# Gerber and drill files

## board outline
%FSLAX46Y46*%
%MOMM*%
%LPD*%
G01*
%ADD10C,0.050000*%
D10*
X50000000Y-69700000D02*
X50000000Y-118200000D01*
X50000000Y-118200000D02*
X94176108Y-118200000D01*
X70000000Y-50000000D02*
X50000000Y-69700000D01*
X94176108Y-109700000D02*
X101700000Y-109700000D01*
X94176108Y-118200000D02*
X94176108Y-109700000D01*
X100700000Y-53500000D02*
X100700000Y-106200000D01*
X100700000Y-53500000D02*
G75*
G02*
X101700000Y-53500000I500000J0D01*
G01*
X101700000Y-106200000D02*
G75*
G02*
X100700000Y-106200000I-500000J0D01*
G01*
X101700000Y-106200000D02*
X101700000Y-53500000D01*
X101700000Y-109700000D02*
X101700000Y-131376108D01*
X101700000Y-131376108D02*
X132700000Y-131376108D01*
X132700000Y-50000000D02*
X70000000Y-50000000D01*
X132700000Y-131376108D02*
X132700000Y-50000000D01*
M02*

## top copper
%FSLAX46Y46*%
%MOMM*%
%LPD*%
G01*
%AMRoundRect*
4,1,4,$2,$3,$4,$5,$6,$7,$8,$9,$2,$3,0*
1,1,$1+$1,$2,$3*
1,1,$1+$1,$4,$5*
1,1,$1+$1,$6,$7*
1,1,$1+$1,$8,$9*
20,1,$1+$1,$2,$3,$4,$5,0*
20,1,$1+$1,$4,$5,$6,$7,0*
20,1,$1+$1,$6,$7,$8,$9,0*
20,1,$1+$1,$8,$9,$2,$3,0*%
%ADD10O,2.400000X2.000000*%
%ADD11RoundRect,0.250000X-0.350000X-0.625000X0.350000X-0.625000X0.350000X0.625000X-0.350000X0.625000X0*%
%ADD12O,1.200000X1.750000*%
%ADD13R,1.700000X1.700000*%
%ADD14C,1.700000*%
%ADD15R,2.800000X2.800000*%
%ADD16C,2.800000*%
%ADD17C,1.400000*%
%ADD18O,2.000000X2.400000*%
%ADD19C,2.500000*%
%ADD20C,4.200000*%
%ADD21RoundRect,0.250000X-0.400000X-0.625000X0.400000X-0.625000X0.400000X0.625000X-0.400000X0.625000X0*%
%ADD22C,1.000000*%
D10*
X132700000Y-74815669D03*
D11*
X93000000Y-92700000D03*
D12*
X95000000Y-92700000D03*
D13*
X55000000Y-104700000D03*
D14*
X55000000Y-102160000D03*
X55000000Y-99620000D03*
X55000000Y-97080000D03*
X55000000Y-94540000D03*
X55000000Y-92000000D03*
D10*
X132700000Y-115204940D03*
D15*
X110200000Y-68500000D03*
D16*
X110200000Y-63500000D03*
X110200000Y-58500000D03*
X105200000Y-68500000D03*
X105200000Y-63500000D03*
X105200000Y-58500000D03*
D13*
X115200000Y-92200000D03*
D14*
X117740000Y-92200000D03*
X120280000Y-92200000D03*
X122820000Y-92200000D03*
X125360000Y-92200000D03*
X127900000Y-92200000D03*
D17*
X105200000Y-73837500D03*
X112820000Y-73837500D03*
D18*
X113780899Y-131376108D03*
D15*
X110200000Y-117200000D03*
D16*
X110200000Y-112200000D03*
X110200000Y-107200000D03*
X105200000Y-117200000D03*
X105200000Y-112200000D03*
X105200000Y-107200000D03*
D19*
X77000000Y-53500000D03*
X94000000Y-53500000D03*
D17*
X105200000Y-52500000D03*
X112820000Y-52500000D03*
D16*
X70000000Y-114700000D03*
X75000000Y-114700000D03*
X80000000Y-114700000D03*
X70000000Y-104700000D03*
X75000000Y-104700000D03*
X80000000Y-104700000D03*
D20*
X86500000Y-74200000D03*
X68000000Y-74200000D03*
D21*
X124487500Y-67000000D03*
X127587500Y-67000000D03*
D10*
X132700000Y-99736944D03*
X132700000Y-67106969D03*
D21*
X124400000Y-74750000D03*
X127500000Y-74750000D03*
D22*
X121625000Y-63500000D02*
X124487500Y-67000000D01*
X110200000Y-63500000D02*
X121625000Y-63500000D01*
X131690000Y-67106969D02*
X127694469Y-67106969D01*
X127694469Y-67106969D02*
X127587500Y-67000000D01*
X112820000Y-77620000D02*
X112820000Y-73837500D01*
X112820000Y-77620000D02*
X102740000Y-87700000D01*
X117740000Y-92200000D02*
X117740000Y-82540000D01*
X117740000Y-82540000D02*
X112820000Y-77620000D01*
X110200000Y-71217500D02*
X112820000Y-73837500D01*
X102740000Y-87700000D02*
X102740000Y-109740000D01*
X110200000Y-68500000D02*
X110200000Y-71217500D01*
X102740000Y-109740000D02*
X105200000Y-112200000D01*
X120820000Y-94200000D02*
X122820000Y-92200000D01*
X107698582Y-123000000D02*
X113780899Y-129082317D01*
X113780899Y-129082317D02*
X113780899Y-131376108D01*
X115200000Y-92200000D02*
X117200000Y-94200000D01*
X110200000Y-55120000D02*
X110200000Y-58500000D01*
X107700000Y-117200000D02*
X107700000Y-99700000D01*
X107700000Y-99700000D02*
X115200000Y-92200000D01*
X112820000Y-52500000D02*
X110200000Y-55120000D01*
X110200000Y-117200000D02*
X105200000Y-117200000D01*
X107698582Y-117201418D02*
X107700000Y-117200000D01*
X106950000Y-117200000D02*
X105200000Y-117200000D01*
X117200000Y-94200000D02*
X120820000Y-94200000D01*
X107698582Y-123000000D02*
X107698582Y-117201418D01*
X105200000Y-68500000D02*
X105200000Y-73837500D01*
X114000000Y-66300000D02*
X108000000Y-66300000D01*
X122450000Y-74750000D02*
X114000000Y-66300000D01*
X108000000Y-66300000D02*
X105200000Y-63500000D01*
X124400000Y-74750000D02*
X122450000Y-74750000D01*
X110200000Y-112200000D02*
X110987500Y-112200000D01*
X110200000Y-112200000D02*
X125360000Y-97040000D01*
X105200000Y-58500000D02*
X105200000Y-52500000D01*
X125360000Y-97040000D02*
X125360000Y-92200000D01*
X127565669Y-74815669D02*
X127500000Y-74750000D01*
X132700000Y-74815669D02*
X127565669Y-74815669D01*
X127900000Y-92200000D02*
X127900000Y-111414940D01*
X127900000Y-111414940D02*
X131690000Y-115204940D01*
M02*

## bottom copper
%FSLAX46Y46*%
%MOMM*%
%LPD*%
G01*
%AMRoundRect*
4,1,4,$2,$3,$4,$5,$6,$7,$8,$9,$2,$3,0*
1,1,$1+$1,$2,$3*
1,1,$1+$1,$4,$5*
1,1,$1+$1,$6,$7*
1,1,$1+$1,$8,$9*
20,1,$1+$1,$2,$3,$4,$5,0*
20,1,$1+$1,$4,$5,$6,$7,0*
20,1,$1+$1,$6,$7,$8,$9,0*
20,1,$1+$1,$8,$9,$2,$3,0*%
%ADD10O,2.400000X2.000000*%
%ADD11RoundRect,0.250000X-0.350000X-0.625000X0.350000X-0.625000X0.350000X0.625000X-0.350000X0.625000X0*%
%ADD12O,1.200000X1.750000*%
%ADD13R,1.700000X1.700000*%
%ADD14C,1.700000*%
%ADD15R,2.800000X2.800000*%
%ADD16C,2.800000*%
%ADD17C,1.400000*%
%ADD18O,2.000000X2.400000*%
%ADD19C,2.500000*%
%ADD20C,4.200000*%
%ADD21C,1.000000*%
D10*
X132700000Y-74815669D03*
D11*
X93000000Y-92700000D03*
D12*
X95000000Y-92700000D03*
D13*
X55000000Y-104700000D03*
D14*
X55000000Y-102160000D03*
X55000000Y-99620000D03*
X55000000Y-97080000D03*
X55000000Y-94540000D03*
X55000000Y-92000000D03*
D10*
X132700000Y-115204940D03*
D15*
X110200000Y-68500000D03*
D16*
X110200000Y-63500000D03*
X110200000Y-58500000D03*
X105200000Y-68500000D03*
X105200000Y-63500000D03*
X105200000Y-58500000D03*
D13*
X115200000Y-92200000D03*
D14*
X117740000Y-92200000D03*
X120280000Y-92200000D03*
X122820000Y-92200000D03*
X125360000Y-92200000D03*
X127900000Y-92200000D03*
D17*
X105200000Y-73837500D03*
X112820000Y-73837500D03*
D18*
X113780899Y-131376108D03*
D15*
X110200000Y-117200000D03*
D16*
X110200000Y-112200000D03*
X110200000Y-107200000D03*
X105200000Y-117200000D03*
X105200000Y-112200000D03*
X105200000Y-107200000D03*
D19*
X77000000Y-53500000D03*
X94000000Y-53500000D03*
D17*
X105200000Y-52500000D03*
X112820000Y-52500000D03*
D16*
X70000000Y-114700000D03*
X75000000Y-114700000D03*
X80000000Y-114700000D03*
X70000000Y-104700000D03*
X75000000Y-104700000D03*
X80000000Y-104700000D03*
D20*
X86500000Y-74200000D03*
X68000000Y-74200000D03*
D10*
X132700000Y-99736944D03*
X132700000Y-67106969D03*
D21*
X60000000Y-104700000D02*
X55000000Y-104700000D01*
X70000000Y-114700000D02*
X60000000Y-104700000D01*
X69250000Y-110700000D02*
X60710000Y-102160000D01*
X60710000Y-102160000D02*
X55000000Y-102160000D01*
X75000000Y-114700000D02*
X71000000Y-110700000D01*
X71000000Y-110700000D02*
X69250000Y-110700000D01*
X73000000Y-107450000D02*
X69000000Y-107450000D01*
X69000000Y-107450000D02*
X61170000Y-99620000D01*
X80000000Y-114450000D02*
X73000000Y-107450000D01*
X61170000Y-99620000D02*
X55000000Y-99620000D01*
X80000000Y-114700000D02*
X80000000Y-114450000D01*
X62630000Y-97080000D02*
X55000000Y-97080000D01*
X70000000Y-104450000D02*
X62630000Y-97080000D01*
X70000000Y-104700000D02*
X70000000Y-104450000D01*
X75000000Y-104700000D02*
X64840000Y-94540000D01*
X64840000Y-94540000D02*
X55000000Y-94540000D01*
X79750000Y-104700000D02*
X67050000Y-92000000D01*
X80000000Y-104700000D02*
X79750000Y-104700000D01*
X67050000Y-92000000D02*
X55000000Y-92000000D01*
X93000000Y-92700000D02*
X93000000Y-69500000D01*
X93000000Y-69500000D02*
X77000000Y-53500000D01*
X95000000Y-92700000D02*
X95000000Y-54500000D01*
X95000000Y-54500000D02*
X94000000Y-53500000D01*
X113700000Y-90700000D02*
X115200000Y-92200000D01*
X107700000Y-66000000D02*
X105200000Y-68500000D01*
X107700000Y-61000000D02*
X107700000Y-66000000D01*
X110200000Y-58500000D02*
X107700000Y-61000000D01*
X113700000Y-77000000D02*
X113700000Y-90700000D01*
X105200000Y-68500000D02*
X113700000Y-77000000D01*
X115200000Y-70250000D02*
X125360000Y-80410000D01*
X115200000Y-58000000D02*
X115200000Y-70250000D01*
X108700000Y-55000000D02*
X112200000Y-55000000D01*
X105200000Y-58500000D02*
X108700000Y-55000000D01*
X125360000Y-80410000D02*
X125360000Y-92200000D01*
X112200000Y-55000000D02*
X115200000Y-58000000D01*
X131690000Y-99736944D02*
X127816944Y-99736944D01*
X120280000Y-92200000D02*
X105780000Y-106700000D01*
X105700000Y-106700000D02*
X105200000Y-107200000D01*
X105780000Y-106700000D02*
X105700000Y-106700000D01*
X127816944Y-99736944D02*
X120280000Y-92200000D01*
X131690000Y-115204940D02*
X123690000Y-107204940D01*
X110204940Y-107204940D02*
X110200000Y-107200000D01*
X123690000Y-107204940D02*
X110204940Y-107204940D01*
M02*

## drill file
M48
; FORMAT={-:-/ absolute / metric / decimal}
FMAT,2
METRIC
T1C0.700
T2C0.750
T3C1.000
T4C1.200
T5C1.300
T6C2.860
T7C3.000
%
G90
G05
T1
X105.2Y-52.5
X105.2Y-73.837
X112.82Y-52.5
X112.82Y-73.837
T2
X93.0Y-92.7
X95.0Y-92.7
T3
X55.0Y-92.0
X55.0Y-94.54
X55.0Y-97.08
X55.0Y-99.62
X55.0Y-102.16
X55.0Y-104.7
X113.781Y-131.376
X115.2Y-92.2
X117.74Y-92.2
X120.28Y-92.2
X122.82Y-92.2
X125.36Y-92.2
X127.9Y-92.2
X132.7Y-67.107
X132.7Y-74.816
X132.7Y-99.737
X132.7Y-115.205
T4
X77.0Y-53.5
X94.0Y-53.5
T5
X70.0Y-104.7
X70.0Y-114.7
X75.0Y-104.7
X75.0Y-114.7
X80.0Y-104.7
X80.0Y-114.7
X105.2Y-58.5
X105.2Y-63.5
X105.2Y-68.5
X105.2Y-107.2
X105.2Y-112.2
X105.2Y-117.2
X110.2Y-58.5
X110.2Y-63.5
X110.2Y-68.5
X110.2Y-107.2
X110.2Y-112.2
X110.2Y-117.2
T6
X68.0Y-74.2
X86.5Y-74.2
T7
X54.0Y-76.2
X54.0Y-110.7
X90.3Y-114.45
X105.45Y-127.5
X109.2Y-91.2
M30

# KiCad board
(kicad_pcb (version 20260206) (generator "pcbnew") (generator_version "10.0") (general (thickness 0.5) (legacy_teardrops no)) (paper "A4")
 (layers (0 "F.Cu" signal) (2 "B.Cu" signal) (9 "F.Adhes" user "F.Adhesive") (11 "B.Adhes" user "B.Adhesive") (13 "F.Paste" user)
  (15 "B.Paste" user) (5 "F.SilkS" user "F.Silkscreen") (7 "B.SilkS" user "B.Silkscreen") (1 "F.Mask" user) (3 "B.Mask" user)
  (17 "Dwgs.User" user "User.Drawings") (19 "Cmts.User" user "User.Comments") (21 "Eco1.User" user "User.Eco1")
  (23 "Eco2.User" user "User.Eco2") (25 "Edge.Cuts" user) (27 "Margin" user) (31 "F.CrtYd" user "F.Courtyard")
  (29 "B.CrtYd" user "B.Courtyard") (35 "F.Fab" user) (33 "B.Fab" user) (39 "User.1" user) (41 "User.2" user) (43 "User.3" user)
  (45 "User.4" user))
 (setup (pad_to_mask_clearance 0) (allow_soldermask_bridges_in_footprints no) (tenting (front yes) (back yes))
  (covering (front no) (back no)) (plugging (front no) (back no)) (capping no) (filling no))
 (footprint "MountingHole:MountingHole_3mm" (layer "F.Cu") (at 54 76.2)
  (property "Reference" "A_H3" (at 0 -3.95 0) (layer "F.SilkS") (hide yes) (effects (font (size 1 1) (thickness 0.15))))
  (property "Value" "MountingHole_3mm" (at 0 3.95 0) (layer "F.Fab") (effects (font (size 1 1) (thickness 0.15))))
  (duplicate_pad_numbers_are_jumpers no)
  (pad "" np_thru_hole circle (at 0 0) (size 3 3) (drill 3) (layers "*.Cu" "*.Mask")))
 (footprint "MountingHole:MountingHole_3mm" (layer "F.Cu") (at 109.2 91.2)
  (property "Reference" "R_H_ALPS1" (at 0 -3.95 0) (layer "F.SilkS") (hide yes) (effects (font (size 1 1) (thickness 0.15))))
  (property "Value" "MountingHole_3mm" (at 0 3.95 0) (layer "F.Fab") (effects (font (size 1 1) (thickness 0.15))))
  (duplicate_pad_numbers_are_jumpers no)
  (pad "" np_thru_hole circle (at 0 0) (size 3 3) (drill 3) (layers "*.Cu" "*.Mask")))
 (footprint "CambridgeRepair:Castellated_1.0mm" (layer "F.Cu") (at 132.7 74.815669)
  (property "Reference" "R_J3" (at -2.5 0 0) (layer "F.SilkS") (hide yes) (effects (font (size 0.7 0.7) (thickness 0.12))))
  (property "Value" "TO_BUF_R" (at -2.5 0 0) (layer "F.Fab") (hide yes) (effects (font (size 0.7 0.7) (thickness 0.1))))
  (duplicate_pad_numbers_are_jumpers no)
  (pad "1" thru_hole oval (at 0 0) (size 2.4 2) (drill 1) (layers "*.Cu" "*.Mask") (remove_unused_layers no) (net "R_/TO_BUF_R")
   (solder_mask_margin 0.05)))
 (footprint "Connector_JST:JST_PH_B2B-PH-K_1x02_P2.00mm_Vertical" (layer "F.Cu") (at 93 92.7)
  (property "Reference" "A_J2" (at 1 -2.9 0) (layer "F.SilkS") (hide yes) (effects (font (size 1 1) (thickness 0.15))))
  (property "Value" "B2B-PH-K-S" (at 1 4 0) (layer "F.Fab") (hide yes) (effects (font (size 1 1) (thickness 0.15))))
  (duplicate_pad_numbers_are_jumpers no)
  (pad "1" thru_hole roundrect (at 0 0) (size 1.2 1.75) (drill 0.75) (layers "*.Cu" "*.Mask") (remove_unused_layers no)
   (roundrect_rratio 0.208333) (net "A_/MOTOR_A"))
  (pad "2" thru_hole oval (at 2 0) (size 1.2 1.75) (drill 0.75) (layers "*.Cu" "*.Mask") (remove_unused_layers no) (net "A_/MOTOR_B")))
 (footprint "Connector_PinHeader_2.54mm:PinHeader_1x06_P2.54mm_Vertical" (layer "F.Cu") (at 55 104.7 180)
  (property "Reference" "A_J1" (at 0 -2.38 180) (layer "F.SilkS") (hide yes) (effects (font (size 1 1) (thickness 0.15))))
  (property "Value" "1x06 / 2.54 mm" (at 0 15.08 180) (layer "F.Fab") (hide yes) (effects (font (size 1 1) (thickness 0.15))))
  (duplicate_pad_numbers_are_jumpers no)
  (pad "1" thru_hole rect (at 0 0 180) (size 1.7 1.7) (drill 1) (layers "*.Cu" "*.Mask") (remove_unused_layers no) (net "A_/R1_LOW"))
  (pad "2" thru_hole circle (at 0 2.54 180) (size 1.7 1.7) (drill 1) (layers "*.Cu" "*.Mask") (remove_unused_layers no) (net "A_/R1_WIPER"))
  (pad "3" thru_hole circle (at 0 5.08 180) (size 1.7 1.7) (drill 1) (layers "*.Cu" "*.Mask") (remove_unused_layers no) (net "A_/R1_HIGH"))
  (pad "4" thru_hole circle (at 0 7.62 180) (size 1.7 1.7) (drill 1) (layers "*.Cu" "*.Mask") (remove_unused_layers no) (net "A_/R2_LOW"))
  (pad "5" thru_hole circle (at 0 10.16 180) (size 1.7 1.7) (drill 1) (layers "*.Cu" "*.Mask") (remove_unused_layers no) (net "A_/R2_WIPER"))
  (pad "6" thru_hole circle (at 0 12.7 180) (size 1.7 1.7) (drill 1) (layers "*.Cu" "*.Mask") (remove_unused_layers no) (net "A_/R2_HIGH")))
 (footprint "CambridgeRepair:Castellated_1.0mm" (layer "F.Cu") (at 132.7 115.20494)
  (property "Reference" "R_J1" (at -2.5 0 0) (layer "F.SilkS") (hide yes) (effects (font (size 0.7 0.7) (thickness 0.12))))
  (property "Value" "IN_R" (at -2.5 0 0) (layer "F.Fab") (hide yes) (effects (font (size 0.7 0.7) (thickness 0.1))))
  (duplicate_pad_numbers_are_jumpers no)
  (pad "1" thru_hole oval (at 0 0) (size 2.4 2) (drill 1) (layers "*.Cu" "*.Mask") (remove_unused_layers no) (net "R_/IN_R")
   (solder_mask_margin 0.05)))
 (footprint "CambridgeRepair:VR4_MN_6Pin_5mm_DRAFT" (layer "F.Cu") (at 105.2 63.5)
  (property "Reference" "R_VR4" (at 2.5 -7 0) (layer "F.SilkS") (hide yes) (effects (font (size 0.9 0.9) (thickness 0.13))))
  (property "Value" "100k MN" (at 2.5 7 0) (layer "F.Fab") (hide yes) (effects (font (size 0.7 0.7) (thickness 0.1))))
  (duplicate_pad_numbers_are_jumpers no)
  (pad "1" thru_hole rect (at 5 5) (size 2.8 2.8) (drill 1.3) (layers "*.Cu" "*.Mask") (remove_unused_layers no) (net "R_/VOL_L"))
  (pad "2" thru_hole circle (at 5 0) (size 2.8 2.8) (drill 1.3) (layers "*.Cu" "*.Mask") (remove_unused_layers no) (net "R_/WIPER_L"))
  (pad "3" thru_hole circle (at 5 -5) (size 2.8 2.8) (drill 1.3) (layers "*.Cu" "*.Mask") (remove_unused_layers no) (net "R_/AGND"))
  (pad "4" thru_hole circle (at 0 5) (size 2.8 2.8) (drill 1.3) (layers "*.Cu" "*.Mask") (remove_unused_layers no) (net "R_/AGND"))
  (pad "5" thru_hole circle (at 0 0) (size 2.8 2.8) (drill 1.3) (layers "*.Cu" "*.Mask") (remove_unused_layers no) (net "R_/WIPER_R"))
  (pad "6" thru_hole circle (at 0 -5) (size 2.8 2.8) (drill 1.3) (layers "*.Cu" "*.Mask") (remove_unused_layers no) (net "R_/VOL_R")))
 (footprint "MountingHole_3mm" (layer "F.Cu") (at 105.45 127.5)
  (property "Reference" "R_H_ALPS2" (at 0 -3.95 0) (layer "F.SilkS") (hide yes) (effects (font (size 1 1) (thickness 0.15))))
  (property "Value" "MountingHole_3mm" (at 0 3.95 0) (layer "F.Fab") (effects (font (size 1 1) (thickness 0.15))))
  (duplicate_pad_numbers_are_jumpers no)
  (pad "" np_thru_hole circle (at 0 0) (size 3 3) (drill 3) (layers "*.Cu" "*.Mask")))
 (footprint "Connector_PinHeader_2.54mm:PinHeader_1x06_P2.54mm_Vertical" (layer "F.Cu") (at 115.2 92.2 90)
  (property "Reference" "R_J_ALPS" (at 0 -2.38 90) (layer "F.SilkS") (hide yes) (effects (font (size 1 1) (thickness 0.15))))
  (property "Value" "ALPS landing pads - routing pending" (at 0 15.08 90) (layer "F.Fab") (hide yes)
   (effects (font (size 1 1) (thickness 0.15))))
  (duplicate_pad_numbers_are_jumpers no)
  (pad "1" thru_hole rect (at 0 0 90) (size 1.7 1.7) (drill 1) (layers "*.Cu" "*.Mask") (remove_unused_layers no) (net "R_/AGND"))
  (pad "2" thru_hole circle (at 0 2.54 90) (size 1.7 1.7) (drill 1) (layers "*.Cu" "*.Mask") (remove_unused_layers no) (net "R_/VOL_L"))
  (pad "3" thru_hole circle (at 0 5.08 90) (size 1.7 1.7) (drill 1) (layers "*.Cu" "*.Mask") (remove_unused_layers no) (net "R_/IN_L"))
  (pad "4" thru_hole circle (at 0 7.62 90) (size 1.7 1.7) (drill 1) (layers "*.Cu" "*.Mask") (remove_unused_layers no) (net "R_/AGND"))
  (pad "5" thru_hole circle (at 0 10.16 90) (size 1.7 1.7) (drill 1) (layers "*.Cu" "*.Mask") (remove_unused_layers no) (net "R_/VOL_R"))
  (pad "6" thru_hole circle (at 0 12.7 90) (size 1.7 1.7) (drill 1) (layers "*.Cu" "*.Mask") (remove_unused_layers no) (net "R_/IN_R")))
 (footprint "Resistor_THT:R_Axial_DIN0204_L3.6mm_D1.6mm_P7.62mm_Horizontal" (layer "F.Cu") (at 105.2 73.8375)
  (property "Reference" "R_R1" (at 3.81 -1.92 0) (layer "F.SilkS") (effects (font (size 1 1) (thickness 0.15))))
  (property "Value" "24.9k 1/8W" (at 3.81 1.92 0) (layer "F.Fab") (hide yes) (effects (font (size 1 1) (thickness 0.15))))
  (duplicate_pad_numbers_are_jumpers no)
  (pad "1" thru_hole circle (at 0 0) (size 1.4 1.4) (drill 0.7) (layers "*.Cu" "*.Mask") (remove_unused_layers no) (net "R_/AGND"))
  (pad "2" thru_hole circle (at 7.62 0) (size 1.4 1.4) (drill 0.7) (layers "*.Cu" "*.Mask") (remove_unused_layers no) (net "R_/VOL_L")))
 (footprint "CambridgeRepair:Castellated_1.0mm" (layer "F.Cu") (at 113.780899 131.376108 90)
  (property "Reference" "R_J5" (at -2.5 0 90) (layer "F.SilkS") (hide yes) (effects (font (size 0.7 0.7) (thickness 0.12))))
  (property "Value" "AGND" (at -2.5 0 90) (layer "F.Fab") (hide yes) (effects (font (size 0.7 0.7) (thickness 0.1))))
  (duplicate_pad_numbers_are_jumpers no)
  (pad "1" thru_hole oval (at 0 0 90) (size 2.4 2) (drill 1) (layers "*.Cu" "*.Mask") (remove_unused_layers no) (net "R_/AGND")
   (solder_mask_margin 0.05)))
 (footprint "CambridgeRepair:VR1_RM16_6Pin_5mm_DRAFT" (layer "F.Cu") (at 105.2 112.2)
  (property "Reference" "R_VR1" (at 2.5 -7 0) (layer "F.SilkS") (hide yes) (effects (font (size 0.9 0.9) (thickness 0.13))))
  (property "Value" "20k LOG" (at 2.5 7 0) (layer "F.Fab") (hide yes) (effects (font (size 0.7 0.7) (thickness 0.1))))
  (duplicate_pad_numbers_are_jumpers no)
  (pad "1" thru_hole rect (at 5 5) (size 2.8 2.8) (drill 1.3) (layers "*.Cu" "*.Mask") (remove_unused_layers no) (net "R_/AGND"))
  (pad "2" thru_hole circle (at 5 0) (size 2.8 2.8) (drill 1.3) (layers "*.Cu" "*.Mask") (remove_unused_layers no) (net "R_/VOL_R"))
  (pad "3" thru_hole circle (at 5 -5) (size 2.8 2.8) (drill 1.3) (layers "*.Cu" "*.Mask") (remove_unused_layers no) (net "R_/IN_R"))
  (pad "4" thru_hole circle (at 0 5) (size 2.8 2.8) (drill 1.3) (layers "*.Cu" "*.Mask") (remove_unused_layers no) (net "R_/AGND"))
  (pad "5" thru_hole circle (at 0 0) (size 2.8 2.8) (drill 1.3) (layers "*.Cu" "*.Mask") (remove_unused_layers no) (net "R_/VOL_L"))
  (pad "6" thru_hole circle (at 0 -5) (size 2.8 2.8) (drill 1.3) (layers "*.Cu" "*.Mask") (remove_unused_layers no) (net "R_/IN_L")))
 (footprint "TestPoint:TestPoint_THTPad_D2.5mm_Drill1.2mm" (layer "F.Cu") (at 77 53.5)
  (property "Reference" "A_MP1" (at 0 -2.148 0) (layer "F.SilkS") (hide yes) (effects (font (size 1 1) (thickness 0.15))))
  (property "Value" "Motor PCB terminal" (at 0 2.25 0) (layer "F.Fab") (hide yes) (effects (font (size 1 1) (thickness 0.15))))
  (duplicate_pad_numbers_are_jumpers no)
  (pad "1" thru_hole circle (at 0 0) (size 2.5 2.5) (drill 1.2) (layers "*.Cu" "*.Mask") (remove_unused_layers no) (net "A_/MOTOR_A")))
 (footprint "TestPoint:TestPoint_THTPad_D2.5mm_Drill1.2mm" (layer "F.Cu") (at 94 53.5)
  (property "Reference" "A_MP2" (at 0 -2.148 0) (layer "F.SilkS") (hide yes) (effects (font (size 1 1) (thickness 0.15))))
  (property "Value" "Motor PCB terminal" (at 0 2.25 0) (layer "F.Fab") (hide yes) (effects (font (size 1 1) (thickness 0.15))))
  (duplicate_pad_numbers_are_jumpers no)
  (pad "1" thru_hole circle (at 0 0) (size 2.5 2.5) (drill 1.2) (layers "*.Cu" "*.Mask") (remove_unused_layers no) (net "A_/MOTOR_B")))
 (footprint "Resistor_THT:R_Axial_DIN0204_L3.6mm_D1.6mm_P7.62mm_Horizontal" (layer "F.Cu") (at 105.2 52.5)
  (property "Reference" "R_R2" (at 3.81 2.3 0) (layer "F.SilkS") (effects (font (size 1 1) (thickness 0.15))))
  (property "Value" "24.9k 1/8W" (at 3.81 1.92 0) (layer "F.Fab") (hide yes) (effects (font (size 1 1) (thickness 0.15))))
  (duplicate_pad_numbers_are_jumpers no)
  (pad "1" thru_hole circle (at 0 0) (size 1.4 1.4) (drill 0.7) (layers "*.Cu" "*.Mask") (remove_unused_layers no) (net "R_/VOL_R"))
  (pad "2" thru_hole circle (at 7.62 0) (size 1.4 1.4) (drill 0.7) (layers "*.Cu" "*.Mask") (remove_unused_layers no) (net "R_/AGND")))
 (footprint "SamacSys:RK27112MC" (layer "F.Cu") (at 75 74.2 -90)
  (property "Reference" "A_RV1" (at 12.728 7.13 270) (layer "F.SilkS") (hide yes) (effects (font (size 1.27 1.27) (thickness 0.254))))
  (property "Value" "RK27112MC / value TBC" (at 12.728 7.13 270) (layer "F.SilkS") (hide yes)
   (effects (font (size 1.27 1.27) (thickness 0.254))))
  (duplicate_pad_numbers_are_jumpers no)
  (pad "1" thru_hole circle (at 40.5 5 270) (size 2.8 2.8) (drill 1.3) (layers "*.Cu" "*.Mask") (remove_unused_layers no) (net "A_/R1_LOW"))
  (pad "2" thru_hole circle (at 40.5 0 270) (size 2.8 2.8) (drill 1.3) (layers "*.Cu" "*.Mask") (remove_unused_layers no)
   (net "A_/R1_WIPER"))
  (pad "3" thru_hole circle (at 40.5 -5 270) (size 2.8 2.8) (drill 1.3) (layers "*.Cu" "*.Mask") (remove_unused_layers no)
   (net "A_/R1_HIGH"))
  (pad "4" thru_hole circle (at 30.5 5 270) (size 2.8 2.8) (drill 1.3) (layers "*.Cu" "*.Mask") (remove_unused_layers no) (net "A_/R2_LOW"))
  (pad "5" thru_hole circle (at 30.5 0 270) (size 2.8 2.8) (drill 1.3) (layers "*.Cu" "*.Mask") (remove_unused_layers no)
   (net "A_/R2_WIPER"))
  (pad "6" thru_hole circle (at 30.5 -5 270) (size 2.8 2.8) (drill 1.3) (layers "*.Cu" "*.Mask") (remove_unused_layers no)
   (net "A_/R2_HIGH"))
  (pad "7" thru_hole circle (at 0 -11.5 270) (size 4.2 4.2) (drill 2.86) (layers "*.Cu" "*.Mask") (remove_unused_layers no)
   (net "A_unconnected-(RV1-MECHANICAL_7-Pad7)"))
  (pad "8" thru_hole circle (at 0 7 270) (size 4.2 4.2) (drill 2.86) (layers "*.Cu" "*.Mask") (remove_unused_layers no)
   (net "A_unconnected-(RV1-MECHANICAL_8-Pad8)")))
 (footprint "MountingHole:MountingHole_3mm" (layer "F.Cu") (at 54 110.7)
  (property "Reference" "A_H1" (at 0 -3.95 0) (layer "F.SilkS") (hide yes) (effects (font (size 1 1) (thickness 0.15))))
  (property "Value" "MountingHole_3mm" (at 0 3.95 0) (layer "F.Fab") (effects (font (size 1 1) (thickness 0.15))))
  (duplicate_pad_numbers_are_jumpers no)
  (pad "" np_thru_hole circle (at 0 0) (size 3 3) (drill 3) (layers "*.Cu" "*.Mask")))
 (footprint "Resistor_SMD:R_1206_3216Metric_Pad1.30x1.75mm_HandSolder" (layer "F.Cu") (at 126.0375 67)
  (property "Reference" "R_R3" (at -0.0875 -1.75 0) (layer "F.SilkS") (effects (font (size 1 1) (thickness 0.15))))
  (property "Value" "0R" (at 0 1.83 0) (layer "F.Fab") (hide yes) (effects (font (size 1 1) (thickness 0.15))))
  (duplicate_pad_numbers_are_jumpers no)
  (pad "1" smd roundrect (at -1.55 0) (size 1.3 1.75) (layers "F.Cu" "F.Mask" "F.Paste") (roundrect_rratio 0.192308) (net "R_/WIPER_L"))
  (pad "2" smd roundrect (at 1.55 0) (size 1.3 1.75) (layers "F.Cu" "F.Mask" "F.Paste") (roundrect_rratio 0.192308) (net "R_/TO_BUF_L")))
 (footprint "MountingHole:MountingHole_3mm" (layer "F.Cu") (at 90.3 114.45)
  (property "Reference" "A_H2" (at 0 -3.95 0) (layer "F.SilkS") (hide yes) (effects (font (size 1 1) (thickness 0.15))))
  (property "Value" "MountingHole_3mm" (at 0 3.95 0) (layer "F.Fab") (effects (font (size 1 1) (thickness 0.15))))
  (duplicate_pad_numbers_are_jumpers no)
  (pad "" np_thru_hole circle (at 0 0) (size 3 3) (drill 3) (layers "*.Cu" "*.Mask")))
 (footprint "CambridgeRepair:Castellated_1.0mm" (layer "F.Cu") (at 132.7 99.736944)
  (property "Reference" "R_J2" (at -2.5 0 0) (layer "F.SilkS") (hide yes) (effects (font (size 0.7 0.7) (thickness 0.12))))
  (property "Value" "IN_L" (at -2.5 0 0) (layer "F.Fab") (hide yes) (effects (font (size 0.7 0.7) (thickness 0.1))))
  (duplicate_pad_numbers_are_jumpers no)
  (pad "1" thru_hole oval (at 0 0) (size 2.4 2) (drill 1) (layers "*.Cu" "*.Mask") (remove_unused_layers no) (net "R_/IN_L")
   (solder_mask_margin 0.05)))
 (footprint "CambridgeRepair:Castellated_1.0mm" (layer "F.Cu") (at 132.7 67.106969)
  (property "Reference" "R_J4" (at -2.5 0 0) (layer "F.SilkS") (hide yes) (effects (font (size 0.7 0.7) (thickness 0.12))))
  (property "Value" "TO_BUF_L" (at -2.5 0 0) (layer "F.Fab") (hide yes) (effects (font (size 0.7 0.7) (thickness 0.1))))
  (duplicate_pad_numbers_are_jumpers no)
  (pad "1" thru_hole oval (at 0 0) (size 2.4 2) (drill 1) (layers "*.Cu" "*.Mask") (remove_unused_layers no) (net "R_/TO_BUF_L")
   (solder_mask_margin 0.05)))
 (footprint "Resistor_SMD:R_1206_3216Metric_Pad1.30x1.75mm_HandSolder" (layer "F.Cu") (at 125.95 74.75)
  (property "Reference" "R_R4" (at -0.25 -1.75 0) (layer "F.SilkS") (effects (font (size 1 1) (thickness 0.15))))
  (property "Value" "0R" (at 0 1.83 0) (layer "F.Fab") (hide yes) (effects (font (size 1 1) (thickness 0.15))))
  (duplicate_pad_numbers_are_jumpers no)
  (pad "1" smd roundrect (at -1.55 0) (size 1.3 1.75) (layers "F.Cu" "F.Mask" "F.Paste") (roundrect_rratio 0.192308) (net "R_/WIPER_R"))
  (pad "2" smd roundrect (at 1.55 0) (size 1.3 1.75) (layers "F.Cu" "F.Mask" "F.Paste") (roundrect_rratio 0.192308) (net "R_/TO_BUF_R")))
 (gr_line (start 50 69.7) (end 50 118.2) (stroke (width 0.05) (type default)) (layer "Edge.Cuts"))
 (gr_line (start 50 118.2) (end 94.176108 118.2) (stroke (width 0.05) (type default)) (layer "Edge.Cuts"))
 (gr_line (start 70 50) (end 50 69.7) (stroke (width 0.05) (type default)) (layer "Edge.Cuts"))
 (gr_line (start 94.176108 109.7) (end 101.7 109.7) (stroke (width 0.05) (type default)) (layer "Edge.Cuts"))
 (gr_line (start 94.176108 118.2) (end 94.176108 109.7) (stroke (width 0.05) (type default)) (layer "Edge.Cuts"))
 (gr_line (start 100.7 53.5) (end 100.7 106.2) (stroke (width 0.05) (type default)) (layer "Edge.Cuts"))
 (gr_arc (start 100.7 53.5) (mid 101.2 53) (end 101.7 53.5) (stroke (width 0.05) (type default)) (layer "Edge.Cuts"))
 (gr_arc (start 101.7 106.2) (mid 101.2 106.7) (end 100.7 106.2) (stroke (width 0.05) (type default)) (layer "Edge.Cuts"))
 (gr_line (start 101.7 106.2) (end 101.7 53.5) (stroke (width 0.05) (type default)) (layer "Edge.Cuts"))
 (gr_line (start 101.7 109.7) (end 101.7 131.376108) (stroke (width 0.05) (type default)) (layer "Edge.Cuts"))
 (gr_line (start 101.7 131.376108) (end 132.7 131.376108) (stroke (width 0.05) (type default)) (layer "Edge.Cuts"))
 (gr_line (start 132.7 50) (end 70 50) (stroke (width 0.05) (type default)) (layer "Edge.Cuts"))
 (gr_line (start 132.7 131.376108) (end 132.7 50) (stroke (width 0.05) (type default)) (layer "Edge.Cuts"))
 (segment (start 60 104.7) (end 55 104.7) (width 1) (layer "B.Cu") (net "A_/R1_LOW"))
 (segment (start 70 114.7) (end 60 104.7) (width 1) (layer "B.Cu") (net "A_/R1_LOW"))
 (segment (start 69.25 110.7) (end 60.71 102.16) (width 1) (layer "B.Cu") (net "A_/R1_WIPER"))
 (segment (start 60.71 102.16) (end 55 102.16) (width 1) (layer "B.Cu") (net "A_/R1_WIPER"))
 (segment (start 75 114.7) (end 71 110.7) (width 1) (layer "B.Cu") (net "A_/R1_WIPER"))
 (segment (start 71 110.7) (end 69.25 110.7) (width 1) (layer "B.Cu") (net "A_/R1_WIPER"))
 (segment (start 73 107.45) (end 69 107.45) (width 1) (layer "B.Cu") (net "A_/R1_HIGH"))
 (segment (start 69 107.45) (end 61.17 99.62) (width 1) (layer "B.Cu") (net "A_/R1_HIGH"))
 (segment (start 80 114.45) (end 73 107.45) (width 1) (layer "B.Cu") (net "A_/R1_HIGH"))
 (segment (start 61.17 99.62) (end 55 99.62) (width 1) (layer "B.Cu") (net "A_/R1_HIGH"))
 (segment (start 80 114.7) (end 80 114.45) (width 1) (layer "B.Cu") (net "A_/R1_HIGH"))
 (segment (start 62.63 97.08) (end 55 97.08) (width 1) (layer "B.Cu") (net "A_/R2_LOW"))
 (segment (start 70 104.45) (end 62.63 97.08) (width 1) (layer "B.Cu") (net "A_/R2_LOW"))
 (segment (start 70 104.7) (end 70 104.45) (width 1) (layer "B.Cu") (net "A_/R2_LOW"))
 (segment (start 75 104.7) (end 64.84 94.54) (width 1) (layer "B.Cu") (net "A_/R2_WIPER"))
 (segment (start 64.84 94.54) (end 55 94.54) (width 1) (layer "B.Cu") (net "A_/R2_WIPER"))
 (segment (start 79.75 104.7) (end 67.05 92) (width 1) (layer "B.Cu") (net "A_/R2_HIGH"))
 (segment (start 80 104.7) (end 79.75 104.7) (width 1) (layer "B.Cu") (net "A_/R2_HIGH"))
 (segment (start 67.05 92) (end 55 92) (width 1) (layer "B.Cu") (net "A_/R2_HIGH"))
 (segment (start 93 92.7) (end 93 69.5) (width 1) (layer "B.Cu") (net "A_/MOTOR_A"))
 (segment (start 93 69.5) (end 77 53.5) (width 1) (layer "B.Cu") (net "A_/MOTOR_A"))
 (segment (start 95 92.7) (end 95 54.5) (width 1) (layer "B.Cu") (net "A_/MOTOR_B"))
 (segment (start 95 54.5) (end 94 53.5) (width 1) (layer "B.Cu") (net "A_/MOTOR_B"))
 (segment (start 121.625 63.5) (end 124.4875 67) (width 1) (layer "F.Cu") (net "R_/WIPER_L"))
 (segment (start 110.2 63.5) (end 121.625 63.5) (width 1) (layer "F.Cu") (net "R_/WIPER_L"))
 (segment (start 131.69 67.106969) (end 127.694469 67.106969) (width 1) (layer "F.Cu") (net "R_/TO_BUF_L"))
 (segment (start 127.694469 67.106969) (end 127.5875 67) (width 1) (layer "F.Cu") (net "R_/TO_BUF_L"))
 (segment (start 112.82 77.62) (end 112.82 73.8375) (width 1) (layer "F.Cu") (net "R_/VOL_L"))
 (segment (start 112.82 77.62) (end 102.74 87.7) (width 1) (layer "F.Cu") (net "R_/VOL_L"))
 (segment (start 117.74 92.2) (end 117.74 82.54) (width 1) (layer "F.Cu") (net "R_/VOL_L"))
 (segment (start 117.74 82.54) (end 112.82 77.62) (width 1) (layer "F.Cu") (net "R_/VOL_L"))
 (segment (start 110.2 71.2175) (end 112.82 73.8375) (width 1) (layer "F.Cu") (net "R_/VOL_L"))
 (segment (start 102.74 87.7) (end 102.74 109.74) (width 1) (layer "F.Cu") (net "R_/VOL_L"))
 (segment (start 110.2 68.5) (end 110.2 71.2175) (width 1) (layer "F.Cu") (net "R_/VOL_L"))
 (segment (start 102.74 109.74) (end 105.2 112.2) (width 1) (layer "F.Cu") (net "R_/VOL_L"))
 (segment (start 120.82 94.2) (end 122.82 92.2) (width 1) (layer "F.Cu") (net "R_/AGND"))
 (segment (start 107.698582 123) (end 113.780899 129.082317) (width 1) (layer "F.Cu") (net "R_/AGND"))
 (segment (start 113.780899 129.082317) (end 113.780899 131.376108) (width 1) (layer "F.Cu") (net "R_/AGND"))
 (segment (start 115.2 92.2) (end 117.2 94.2) (width 1) (layer "F.Cu") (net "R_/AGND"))
 (segment (start 110.2 55.12) (end 110.2 58.5) (width 1) (layer "F.Cu") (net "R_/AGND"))
 (segment (start 107.7 117.2) (end 107.7 99.7) (width 1) (layer "F.Cu") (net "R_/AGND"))
 (segment (start 107.7 99.7) (end 115.2 92.2) (width 1) (layer "F.Cu") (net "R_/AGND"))
 (segment (start 112.82 52.5) (end 110.2 55.12) (width 1) (layer "F.Cu") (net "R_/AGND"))
 (segment (start 110.2 117.2) (end 105.2 117.2) (width 1) (layer "F.Cu") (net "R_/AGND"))
 (segment (start 107.698582 117.201418) (end 107.7 117.2) (width 1) (layer "F.Cu") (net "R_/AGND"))
 (segment (start 106.95 117.2) (end 105.2 117.2) (width 1) (layer "F.Cu") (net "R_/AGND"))
 (segment (start 117.2 94.2) (end 120.82 94.2) (width 1) (layer "F.Cu") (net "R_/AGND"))
 (segment (start 107.698582 123) (end 107.698582 117.201418) (width 1) (layer "F.Cu") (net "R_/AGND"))
 (segment (start 105.2 68.5) (end 105.2 73.8375) (width 1) (layer "F.Cu") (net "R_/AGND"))
 (segment (start 113.7 90.7) (end 115.2 92.2) (width 1) (layer "B.Cu") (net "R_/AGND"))
 (segment (start 107.7 66) (end 105.2 68.5) (width 1) (layer "B.Cu") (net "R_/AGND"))
 (segment (start 107.7 61) (end 107.7 66) (width 1) (layer "B.Cu") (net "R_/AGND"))
 (segment (start 110.2 58.5) (end 107.7 61) (width 1) (layer "B.Cu") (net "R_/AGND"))
 (segment (start 113.7 77) (end 113.7 90.7) (width 1) (layer "B.Cu") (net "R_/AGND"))
 (segment (start 105.2 68.5) (end 113.7 77) (width 1) (layer "B.Cu") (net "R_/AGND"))
 (segment (start 114 66.3) (end 108 66.3) (width 1) (layer "F.Cu") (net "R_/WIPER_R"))
 (segment (start 122.45 74.75) (end 114 66.3) (width 1) (layer "F.Cu") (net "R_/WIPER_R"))
 (segment (start 108 66.3) (end 105.2 63.5) (width 1) (layer "F.Cu") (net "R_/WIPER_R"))
 (segment (start 124.4 74.75) (end 122.45 74.75) (width 1) (layer "F.Cu") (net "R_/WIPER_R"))
 (segment (start 110.2 112.2) (end 110.9875 112.2) (width 1) (layer "F.Cu") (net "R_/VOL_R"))
 (segment (start 110.2 112.2) (end 125.36 97.04) (width 1) (layer "F.Cu") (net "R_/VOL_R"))
 (segment (start 105.2 58.5) (end 105.2 52.5) (width 1) (layer "F.Cu") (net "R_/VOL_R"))
 (segment (start 125.36 97.04) (end 125.36 92.2) (width 1) (layer "F.Cu") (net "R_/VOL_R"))
 (segment (start 115.2 70.25) (end 125.36 80.41) (width 1) (layer "B.Cu") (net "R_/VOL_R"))
 (segment (start 115.2 58) (end 115.2 70.25) (width 1) (layer "B.Cu") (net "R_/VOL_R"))
 (segment (start 108.7 55) (end 112.2 55) (width 1) (layer "B.Cu") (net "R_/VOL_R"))
 (segment (start 105.2 58.5) (end 108.7 55) (width 1) (layer "B.Cu") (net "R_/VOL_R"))
 (segment (start 125.36 80.41) (end 125.36 92.2) (width 1) (layer "B.Cu") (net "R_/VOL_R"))
 (segment (start 112.2 55) (end 115.2 58) (width 1) (layer "B.Cu") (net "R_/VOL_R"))
 (segment (start 127.565669 74.815669) (end 127.5 74.75) (width 1) (layer "F.Cu") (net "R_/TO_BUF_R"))
 (segment (start 132.7 74.815669) (end 127.565669 74.815669) (width 1) (layer "F.Cu") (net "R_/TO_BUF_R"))
 (segment (start 131.69 99.736944) (end 127.816944 99.736944) (width 1) (layer "B.Cu") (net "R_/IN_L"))
 (segment (start 120.28 92.2) (end 105.78 106.7) (width 1) (layer "B.Cu") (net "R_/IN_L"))
 (segment (start 105.7 106.7) (end 105.2 107.2) (width 1) (layer "B.Cu") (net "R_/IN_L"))
 (segment (start 105.78 106.7) (end 105.7 106.7) (width 1) (layer "B.Cu") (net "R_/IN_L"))
 (segment (start 127.816944 99.736944) (end 120.28 92.2) (width 1) (layer "B.Cu") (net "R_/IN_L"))
 (segment (start 127.9 92.2) (end 127.9 111.41494) (width 1) (layer "F.Cu") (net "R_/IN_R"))
 (segment (start 127.9 111.41494) (end 131.69 115.20494) (width 1) (layer "F.Cu") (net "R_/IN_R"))
 (segment (start 131.69 115.20494) (end 123.69 107.20494) (width 1) (layer "B.Cu") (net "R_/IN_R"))
 (segment (start 110.20494 107.20494) (end 110.2 107.2) (width 1) (layer "B.Cu") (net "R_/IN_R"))
 (segment (start 123.69 107.20494) (end 110.20494 107.20494) (width 1) (layer "B.Cu") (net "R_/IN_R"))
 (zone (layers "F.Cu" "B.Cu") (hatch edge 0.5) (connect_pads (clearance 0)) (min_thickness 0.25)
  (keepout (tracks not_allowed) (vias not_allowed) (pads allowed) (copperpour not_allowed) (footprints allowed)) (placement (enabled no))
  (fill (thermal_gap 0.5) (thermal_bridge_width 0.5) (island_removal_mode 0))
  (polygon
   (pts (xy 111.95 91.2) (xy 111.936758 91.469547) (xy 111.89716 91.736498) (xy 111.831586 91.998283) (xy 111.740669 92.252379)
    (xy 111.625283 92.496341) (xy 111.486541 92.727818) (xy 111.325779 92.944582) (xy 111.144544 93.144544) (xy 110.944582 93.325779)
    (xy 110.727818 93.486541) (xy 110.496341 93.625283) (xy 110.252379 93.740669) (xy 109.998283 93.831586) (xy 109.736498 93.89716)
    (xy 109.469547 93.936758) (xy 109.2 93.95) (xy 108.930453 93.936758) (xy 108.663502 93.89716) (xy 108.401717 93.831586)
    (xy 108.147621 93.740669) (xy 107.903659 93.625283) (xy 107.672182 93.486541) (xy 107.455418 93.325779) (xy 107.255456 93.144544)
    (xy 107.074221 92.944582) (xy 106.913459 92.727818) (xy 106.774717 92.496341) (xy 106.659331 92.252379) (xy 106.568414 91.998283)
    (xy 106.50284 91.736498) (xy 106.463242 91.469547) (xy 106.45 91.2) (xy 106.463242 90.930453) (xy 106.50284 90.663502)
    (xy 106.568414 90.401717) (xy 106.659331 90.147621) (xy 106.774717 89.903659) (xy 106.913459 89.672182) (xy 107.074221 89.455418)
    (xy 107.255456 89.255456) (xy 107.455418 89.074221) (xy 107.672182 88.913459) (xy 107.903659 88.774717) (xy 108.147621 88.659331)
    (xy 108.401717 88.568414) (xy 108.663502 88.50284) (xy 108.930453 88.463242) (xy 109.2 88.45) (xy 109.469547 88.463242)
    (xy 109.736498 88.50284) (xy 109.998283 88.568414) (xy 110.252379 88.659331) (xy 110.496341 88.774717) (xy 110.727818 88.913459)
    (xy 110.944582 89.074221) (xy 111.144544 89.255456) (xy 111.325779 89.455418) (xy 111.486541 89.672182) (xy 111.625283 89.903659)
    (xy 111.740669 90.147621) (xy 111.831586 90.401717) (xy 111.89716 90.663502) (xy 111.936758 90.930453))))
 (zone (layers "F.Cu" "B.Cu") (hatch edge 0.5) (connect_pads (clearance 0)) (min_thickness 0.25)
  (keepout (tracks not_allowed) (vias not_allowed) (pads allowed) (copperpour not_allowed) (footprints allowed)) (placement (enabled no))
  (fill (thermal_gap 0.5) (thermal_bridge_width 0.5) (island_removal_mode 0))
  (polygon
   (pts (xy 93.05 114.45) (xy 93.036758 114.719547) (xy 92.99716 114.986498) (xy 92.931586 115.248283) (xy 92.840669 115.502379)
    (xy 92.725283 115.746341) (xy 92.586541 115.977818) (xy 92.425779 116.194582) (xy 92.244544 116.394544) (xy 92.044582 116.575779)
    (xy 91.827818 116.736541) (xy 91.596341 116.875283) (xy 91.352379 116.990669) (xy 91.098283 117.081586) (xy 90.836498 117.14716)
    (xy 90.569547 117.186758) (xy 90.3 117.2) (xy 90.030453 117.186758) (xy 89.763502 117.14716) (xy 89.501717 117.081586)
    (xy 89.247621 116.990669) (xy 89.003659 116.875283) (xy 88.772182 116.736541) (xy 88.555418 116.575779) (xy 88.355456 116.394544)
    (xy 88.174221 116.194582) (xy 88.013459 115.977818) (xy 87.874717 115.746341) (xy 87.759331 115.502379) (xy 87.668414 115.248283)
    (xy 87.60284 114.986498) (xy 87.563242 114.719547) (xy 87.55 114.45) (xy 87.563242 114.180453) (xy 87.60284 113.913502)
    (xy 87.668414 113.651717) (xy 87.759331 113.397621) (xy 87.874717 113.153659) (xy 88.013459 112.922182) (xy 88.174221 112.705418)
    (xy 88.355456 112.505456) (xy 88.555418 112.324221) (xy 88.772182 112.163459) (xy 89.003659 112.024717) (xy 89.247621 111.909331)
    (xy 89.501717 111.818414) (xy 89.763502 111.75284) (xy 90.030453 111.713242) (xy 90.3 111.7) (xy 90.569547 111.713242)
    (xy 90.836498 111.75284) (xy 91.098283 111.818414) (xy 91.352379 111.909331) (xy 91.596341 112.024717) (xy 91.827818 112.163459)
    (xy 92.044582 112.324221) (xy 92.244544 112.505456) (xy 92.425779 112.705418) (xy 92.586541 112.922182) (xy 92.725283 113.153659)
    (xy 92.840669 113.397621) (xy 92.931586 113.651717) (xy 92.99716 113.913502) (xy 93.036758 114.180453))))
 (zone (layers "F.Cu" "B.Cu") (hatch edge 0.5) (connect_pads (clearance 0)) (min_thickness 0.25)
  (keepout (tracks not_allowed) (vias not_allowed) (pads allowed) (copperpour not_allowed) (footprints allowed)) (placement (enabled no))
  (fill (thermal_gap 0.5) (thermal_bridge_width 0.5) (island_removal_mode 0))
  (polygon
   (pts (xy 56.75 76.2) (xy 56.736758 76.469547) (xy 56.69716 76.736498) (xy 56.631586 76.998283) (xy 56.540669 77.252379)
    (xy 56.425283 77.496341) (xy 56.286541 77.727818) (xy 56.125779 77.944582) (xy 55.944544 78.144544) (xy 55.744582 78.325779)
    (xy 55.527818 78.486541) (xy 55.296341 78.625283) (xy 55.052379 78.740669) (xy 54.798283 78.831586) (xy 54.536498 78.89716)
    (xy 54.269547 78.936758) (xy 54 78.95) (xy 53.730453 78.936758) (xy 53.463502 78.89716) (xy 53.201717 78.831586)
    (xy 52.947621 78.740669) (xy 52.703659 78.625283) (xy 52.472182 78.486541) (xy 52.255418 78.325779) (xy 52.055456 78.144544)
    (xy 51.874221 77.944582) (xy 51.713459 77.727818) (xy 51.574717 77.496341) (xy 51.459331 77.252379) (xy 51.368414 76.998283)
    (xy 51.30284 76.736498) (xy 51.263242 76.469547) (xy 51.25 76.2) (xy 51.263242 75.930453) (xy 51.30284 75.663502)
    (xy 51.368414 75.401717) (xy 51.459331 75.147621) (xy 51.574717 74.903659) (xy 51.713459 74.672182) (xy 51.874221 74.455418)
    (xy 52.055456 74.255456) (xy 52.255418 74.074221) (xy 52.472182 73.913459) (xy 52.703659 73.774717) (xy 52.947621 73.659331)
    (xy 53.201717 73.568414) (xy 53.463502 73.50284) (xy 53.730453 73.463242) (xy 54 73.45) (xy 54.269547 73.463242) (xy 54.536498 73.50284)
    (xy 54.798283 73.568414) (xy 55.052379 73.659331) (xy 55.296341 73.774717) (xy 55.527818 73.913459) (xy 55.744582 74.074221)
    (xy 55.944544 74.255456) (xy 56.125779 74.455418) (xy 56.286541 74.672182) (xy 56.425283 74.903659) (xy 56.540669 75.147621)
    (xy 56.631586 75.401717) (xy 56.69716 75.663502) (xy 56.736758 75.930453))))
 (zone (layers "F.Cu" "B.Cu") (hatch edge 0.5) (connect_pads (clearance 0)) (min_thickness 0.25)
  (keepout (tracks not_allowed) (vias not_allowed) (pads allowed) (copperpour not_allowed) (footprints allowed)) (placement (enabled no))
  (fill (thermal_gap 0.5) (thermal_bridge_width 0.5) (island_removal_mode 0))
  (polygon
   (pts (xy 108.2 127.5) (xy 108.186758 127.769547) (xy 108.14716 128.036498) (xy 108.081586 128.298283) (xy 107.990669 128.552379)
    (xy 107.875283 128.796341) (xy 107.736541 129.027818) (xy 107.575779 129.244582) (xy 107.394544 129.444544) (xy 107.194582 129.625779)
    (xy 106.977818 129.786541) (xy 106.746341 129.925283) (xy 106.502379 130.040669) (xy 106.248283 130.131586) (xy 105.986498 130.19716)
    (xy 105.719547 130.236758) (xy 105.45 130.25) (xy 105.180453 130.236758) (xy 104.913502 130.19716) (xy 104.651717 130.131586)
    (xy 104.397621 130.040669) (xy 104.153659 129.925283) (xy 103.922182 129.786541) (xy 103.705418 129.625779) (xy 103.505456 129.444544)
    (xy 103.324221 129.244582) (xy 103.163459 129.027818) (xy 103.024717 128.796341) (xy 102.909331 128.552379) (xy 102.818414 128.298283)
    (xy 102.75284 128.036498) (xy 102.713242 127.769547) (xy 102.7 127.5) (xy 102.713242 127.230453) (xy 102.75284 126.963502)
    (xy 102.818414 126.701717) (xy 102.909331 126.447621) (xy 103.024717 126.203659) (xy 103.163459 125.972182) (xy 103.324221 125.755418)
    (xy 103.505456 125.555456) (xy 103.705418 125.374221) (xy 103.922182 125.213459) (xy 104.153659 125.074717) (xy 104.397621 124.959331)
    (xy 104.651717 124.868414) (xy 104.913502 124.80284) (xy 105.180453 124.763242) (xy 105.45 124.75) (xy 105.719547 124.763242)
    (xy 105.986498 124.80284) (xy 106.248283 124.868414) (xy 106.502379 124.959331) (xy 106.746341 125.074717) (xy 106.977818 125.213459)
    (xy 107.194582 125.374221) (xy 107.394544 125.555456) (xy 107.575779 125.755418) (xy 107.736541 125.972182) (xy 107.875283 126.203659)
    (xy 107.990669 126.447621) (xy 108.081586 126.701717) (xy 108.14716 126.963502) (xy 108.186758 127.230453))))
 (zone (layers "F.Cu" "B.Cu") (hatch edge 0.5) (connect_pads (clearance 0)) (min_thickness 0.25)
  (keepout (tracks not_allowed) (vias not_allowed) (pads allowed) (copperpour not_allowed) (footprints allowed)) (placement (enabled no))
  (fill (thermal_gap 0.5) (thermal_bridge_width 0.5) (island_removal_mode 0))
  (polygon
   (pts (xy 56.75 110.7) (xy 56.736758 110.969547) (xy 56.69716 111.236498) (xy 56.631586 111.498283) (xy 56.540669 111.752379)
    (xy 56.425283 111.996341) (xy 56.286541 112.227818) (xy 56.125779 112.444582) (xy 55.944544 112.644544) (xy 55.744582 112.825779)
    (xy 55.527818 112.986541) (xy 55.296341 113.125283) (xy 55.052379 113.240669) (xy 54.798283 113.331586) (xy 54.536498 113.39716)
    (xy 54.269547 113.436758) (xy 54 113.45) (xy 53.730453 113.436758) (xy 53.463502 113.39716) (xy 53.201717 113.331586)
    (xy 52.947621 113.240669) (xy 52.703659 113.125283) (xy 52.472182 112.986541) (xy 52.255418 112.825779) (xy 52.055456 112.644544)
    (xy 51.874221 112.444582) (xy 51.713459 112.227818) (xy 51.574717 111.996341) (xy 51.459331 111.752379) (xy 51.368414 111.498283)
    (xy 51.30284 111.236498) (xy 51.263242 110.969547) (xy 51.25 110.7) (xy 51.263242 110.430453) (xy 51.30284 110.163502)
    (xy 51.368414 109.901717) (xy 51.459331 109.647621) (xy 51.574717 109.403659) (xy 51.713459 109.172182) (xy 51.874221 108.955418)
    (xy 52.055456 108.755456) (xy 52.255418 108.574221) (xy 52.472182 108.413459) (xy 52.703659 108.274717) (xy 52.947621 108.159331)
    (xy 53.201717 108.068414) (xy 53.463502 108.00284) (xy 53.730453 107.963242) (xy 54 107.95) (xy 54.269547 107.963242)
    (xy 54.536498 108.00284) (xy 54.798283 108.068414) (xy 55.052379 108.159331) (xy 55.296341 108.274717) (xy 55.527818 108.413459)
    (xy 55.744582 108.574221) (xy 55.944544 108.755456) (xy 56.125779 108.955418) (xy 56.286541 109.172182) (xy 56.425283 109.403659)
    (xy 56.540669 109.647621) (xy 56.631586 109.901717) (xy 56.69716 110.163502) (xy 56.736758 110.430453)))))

